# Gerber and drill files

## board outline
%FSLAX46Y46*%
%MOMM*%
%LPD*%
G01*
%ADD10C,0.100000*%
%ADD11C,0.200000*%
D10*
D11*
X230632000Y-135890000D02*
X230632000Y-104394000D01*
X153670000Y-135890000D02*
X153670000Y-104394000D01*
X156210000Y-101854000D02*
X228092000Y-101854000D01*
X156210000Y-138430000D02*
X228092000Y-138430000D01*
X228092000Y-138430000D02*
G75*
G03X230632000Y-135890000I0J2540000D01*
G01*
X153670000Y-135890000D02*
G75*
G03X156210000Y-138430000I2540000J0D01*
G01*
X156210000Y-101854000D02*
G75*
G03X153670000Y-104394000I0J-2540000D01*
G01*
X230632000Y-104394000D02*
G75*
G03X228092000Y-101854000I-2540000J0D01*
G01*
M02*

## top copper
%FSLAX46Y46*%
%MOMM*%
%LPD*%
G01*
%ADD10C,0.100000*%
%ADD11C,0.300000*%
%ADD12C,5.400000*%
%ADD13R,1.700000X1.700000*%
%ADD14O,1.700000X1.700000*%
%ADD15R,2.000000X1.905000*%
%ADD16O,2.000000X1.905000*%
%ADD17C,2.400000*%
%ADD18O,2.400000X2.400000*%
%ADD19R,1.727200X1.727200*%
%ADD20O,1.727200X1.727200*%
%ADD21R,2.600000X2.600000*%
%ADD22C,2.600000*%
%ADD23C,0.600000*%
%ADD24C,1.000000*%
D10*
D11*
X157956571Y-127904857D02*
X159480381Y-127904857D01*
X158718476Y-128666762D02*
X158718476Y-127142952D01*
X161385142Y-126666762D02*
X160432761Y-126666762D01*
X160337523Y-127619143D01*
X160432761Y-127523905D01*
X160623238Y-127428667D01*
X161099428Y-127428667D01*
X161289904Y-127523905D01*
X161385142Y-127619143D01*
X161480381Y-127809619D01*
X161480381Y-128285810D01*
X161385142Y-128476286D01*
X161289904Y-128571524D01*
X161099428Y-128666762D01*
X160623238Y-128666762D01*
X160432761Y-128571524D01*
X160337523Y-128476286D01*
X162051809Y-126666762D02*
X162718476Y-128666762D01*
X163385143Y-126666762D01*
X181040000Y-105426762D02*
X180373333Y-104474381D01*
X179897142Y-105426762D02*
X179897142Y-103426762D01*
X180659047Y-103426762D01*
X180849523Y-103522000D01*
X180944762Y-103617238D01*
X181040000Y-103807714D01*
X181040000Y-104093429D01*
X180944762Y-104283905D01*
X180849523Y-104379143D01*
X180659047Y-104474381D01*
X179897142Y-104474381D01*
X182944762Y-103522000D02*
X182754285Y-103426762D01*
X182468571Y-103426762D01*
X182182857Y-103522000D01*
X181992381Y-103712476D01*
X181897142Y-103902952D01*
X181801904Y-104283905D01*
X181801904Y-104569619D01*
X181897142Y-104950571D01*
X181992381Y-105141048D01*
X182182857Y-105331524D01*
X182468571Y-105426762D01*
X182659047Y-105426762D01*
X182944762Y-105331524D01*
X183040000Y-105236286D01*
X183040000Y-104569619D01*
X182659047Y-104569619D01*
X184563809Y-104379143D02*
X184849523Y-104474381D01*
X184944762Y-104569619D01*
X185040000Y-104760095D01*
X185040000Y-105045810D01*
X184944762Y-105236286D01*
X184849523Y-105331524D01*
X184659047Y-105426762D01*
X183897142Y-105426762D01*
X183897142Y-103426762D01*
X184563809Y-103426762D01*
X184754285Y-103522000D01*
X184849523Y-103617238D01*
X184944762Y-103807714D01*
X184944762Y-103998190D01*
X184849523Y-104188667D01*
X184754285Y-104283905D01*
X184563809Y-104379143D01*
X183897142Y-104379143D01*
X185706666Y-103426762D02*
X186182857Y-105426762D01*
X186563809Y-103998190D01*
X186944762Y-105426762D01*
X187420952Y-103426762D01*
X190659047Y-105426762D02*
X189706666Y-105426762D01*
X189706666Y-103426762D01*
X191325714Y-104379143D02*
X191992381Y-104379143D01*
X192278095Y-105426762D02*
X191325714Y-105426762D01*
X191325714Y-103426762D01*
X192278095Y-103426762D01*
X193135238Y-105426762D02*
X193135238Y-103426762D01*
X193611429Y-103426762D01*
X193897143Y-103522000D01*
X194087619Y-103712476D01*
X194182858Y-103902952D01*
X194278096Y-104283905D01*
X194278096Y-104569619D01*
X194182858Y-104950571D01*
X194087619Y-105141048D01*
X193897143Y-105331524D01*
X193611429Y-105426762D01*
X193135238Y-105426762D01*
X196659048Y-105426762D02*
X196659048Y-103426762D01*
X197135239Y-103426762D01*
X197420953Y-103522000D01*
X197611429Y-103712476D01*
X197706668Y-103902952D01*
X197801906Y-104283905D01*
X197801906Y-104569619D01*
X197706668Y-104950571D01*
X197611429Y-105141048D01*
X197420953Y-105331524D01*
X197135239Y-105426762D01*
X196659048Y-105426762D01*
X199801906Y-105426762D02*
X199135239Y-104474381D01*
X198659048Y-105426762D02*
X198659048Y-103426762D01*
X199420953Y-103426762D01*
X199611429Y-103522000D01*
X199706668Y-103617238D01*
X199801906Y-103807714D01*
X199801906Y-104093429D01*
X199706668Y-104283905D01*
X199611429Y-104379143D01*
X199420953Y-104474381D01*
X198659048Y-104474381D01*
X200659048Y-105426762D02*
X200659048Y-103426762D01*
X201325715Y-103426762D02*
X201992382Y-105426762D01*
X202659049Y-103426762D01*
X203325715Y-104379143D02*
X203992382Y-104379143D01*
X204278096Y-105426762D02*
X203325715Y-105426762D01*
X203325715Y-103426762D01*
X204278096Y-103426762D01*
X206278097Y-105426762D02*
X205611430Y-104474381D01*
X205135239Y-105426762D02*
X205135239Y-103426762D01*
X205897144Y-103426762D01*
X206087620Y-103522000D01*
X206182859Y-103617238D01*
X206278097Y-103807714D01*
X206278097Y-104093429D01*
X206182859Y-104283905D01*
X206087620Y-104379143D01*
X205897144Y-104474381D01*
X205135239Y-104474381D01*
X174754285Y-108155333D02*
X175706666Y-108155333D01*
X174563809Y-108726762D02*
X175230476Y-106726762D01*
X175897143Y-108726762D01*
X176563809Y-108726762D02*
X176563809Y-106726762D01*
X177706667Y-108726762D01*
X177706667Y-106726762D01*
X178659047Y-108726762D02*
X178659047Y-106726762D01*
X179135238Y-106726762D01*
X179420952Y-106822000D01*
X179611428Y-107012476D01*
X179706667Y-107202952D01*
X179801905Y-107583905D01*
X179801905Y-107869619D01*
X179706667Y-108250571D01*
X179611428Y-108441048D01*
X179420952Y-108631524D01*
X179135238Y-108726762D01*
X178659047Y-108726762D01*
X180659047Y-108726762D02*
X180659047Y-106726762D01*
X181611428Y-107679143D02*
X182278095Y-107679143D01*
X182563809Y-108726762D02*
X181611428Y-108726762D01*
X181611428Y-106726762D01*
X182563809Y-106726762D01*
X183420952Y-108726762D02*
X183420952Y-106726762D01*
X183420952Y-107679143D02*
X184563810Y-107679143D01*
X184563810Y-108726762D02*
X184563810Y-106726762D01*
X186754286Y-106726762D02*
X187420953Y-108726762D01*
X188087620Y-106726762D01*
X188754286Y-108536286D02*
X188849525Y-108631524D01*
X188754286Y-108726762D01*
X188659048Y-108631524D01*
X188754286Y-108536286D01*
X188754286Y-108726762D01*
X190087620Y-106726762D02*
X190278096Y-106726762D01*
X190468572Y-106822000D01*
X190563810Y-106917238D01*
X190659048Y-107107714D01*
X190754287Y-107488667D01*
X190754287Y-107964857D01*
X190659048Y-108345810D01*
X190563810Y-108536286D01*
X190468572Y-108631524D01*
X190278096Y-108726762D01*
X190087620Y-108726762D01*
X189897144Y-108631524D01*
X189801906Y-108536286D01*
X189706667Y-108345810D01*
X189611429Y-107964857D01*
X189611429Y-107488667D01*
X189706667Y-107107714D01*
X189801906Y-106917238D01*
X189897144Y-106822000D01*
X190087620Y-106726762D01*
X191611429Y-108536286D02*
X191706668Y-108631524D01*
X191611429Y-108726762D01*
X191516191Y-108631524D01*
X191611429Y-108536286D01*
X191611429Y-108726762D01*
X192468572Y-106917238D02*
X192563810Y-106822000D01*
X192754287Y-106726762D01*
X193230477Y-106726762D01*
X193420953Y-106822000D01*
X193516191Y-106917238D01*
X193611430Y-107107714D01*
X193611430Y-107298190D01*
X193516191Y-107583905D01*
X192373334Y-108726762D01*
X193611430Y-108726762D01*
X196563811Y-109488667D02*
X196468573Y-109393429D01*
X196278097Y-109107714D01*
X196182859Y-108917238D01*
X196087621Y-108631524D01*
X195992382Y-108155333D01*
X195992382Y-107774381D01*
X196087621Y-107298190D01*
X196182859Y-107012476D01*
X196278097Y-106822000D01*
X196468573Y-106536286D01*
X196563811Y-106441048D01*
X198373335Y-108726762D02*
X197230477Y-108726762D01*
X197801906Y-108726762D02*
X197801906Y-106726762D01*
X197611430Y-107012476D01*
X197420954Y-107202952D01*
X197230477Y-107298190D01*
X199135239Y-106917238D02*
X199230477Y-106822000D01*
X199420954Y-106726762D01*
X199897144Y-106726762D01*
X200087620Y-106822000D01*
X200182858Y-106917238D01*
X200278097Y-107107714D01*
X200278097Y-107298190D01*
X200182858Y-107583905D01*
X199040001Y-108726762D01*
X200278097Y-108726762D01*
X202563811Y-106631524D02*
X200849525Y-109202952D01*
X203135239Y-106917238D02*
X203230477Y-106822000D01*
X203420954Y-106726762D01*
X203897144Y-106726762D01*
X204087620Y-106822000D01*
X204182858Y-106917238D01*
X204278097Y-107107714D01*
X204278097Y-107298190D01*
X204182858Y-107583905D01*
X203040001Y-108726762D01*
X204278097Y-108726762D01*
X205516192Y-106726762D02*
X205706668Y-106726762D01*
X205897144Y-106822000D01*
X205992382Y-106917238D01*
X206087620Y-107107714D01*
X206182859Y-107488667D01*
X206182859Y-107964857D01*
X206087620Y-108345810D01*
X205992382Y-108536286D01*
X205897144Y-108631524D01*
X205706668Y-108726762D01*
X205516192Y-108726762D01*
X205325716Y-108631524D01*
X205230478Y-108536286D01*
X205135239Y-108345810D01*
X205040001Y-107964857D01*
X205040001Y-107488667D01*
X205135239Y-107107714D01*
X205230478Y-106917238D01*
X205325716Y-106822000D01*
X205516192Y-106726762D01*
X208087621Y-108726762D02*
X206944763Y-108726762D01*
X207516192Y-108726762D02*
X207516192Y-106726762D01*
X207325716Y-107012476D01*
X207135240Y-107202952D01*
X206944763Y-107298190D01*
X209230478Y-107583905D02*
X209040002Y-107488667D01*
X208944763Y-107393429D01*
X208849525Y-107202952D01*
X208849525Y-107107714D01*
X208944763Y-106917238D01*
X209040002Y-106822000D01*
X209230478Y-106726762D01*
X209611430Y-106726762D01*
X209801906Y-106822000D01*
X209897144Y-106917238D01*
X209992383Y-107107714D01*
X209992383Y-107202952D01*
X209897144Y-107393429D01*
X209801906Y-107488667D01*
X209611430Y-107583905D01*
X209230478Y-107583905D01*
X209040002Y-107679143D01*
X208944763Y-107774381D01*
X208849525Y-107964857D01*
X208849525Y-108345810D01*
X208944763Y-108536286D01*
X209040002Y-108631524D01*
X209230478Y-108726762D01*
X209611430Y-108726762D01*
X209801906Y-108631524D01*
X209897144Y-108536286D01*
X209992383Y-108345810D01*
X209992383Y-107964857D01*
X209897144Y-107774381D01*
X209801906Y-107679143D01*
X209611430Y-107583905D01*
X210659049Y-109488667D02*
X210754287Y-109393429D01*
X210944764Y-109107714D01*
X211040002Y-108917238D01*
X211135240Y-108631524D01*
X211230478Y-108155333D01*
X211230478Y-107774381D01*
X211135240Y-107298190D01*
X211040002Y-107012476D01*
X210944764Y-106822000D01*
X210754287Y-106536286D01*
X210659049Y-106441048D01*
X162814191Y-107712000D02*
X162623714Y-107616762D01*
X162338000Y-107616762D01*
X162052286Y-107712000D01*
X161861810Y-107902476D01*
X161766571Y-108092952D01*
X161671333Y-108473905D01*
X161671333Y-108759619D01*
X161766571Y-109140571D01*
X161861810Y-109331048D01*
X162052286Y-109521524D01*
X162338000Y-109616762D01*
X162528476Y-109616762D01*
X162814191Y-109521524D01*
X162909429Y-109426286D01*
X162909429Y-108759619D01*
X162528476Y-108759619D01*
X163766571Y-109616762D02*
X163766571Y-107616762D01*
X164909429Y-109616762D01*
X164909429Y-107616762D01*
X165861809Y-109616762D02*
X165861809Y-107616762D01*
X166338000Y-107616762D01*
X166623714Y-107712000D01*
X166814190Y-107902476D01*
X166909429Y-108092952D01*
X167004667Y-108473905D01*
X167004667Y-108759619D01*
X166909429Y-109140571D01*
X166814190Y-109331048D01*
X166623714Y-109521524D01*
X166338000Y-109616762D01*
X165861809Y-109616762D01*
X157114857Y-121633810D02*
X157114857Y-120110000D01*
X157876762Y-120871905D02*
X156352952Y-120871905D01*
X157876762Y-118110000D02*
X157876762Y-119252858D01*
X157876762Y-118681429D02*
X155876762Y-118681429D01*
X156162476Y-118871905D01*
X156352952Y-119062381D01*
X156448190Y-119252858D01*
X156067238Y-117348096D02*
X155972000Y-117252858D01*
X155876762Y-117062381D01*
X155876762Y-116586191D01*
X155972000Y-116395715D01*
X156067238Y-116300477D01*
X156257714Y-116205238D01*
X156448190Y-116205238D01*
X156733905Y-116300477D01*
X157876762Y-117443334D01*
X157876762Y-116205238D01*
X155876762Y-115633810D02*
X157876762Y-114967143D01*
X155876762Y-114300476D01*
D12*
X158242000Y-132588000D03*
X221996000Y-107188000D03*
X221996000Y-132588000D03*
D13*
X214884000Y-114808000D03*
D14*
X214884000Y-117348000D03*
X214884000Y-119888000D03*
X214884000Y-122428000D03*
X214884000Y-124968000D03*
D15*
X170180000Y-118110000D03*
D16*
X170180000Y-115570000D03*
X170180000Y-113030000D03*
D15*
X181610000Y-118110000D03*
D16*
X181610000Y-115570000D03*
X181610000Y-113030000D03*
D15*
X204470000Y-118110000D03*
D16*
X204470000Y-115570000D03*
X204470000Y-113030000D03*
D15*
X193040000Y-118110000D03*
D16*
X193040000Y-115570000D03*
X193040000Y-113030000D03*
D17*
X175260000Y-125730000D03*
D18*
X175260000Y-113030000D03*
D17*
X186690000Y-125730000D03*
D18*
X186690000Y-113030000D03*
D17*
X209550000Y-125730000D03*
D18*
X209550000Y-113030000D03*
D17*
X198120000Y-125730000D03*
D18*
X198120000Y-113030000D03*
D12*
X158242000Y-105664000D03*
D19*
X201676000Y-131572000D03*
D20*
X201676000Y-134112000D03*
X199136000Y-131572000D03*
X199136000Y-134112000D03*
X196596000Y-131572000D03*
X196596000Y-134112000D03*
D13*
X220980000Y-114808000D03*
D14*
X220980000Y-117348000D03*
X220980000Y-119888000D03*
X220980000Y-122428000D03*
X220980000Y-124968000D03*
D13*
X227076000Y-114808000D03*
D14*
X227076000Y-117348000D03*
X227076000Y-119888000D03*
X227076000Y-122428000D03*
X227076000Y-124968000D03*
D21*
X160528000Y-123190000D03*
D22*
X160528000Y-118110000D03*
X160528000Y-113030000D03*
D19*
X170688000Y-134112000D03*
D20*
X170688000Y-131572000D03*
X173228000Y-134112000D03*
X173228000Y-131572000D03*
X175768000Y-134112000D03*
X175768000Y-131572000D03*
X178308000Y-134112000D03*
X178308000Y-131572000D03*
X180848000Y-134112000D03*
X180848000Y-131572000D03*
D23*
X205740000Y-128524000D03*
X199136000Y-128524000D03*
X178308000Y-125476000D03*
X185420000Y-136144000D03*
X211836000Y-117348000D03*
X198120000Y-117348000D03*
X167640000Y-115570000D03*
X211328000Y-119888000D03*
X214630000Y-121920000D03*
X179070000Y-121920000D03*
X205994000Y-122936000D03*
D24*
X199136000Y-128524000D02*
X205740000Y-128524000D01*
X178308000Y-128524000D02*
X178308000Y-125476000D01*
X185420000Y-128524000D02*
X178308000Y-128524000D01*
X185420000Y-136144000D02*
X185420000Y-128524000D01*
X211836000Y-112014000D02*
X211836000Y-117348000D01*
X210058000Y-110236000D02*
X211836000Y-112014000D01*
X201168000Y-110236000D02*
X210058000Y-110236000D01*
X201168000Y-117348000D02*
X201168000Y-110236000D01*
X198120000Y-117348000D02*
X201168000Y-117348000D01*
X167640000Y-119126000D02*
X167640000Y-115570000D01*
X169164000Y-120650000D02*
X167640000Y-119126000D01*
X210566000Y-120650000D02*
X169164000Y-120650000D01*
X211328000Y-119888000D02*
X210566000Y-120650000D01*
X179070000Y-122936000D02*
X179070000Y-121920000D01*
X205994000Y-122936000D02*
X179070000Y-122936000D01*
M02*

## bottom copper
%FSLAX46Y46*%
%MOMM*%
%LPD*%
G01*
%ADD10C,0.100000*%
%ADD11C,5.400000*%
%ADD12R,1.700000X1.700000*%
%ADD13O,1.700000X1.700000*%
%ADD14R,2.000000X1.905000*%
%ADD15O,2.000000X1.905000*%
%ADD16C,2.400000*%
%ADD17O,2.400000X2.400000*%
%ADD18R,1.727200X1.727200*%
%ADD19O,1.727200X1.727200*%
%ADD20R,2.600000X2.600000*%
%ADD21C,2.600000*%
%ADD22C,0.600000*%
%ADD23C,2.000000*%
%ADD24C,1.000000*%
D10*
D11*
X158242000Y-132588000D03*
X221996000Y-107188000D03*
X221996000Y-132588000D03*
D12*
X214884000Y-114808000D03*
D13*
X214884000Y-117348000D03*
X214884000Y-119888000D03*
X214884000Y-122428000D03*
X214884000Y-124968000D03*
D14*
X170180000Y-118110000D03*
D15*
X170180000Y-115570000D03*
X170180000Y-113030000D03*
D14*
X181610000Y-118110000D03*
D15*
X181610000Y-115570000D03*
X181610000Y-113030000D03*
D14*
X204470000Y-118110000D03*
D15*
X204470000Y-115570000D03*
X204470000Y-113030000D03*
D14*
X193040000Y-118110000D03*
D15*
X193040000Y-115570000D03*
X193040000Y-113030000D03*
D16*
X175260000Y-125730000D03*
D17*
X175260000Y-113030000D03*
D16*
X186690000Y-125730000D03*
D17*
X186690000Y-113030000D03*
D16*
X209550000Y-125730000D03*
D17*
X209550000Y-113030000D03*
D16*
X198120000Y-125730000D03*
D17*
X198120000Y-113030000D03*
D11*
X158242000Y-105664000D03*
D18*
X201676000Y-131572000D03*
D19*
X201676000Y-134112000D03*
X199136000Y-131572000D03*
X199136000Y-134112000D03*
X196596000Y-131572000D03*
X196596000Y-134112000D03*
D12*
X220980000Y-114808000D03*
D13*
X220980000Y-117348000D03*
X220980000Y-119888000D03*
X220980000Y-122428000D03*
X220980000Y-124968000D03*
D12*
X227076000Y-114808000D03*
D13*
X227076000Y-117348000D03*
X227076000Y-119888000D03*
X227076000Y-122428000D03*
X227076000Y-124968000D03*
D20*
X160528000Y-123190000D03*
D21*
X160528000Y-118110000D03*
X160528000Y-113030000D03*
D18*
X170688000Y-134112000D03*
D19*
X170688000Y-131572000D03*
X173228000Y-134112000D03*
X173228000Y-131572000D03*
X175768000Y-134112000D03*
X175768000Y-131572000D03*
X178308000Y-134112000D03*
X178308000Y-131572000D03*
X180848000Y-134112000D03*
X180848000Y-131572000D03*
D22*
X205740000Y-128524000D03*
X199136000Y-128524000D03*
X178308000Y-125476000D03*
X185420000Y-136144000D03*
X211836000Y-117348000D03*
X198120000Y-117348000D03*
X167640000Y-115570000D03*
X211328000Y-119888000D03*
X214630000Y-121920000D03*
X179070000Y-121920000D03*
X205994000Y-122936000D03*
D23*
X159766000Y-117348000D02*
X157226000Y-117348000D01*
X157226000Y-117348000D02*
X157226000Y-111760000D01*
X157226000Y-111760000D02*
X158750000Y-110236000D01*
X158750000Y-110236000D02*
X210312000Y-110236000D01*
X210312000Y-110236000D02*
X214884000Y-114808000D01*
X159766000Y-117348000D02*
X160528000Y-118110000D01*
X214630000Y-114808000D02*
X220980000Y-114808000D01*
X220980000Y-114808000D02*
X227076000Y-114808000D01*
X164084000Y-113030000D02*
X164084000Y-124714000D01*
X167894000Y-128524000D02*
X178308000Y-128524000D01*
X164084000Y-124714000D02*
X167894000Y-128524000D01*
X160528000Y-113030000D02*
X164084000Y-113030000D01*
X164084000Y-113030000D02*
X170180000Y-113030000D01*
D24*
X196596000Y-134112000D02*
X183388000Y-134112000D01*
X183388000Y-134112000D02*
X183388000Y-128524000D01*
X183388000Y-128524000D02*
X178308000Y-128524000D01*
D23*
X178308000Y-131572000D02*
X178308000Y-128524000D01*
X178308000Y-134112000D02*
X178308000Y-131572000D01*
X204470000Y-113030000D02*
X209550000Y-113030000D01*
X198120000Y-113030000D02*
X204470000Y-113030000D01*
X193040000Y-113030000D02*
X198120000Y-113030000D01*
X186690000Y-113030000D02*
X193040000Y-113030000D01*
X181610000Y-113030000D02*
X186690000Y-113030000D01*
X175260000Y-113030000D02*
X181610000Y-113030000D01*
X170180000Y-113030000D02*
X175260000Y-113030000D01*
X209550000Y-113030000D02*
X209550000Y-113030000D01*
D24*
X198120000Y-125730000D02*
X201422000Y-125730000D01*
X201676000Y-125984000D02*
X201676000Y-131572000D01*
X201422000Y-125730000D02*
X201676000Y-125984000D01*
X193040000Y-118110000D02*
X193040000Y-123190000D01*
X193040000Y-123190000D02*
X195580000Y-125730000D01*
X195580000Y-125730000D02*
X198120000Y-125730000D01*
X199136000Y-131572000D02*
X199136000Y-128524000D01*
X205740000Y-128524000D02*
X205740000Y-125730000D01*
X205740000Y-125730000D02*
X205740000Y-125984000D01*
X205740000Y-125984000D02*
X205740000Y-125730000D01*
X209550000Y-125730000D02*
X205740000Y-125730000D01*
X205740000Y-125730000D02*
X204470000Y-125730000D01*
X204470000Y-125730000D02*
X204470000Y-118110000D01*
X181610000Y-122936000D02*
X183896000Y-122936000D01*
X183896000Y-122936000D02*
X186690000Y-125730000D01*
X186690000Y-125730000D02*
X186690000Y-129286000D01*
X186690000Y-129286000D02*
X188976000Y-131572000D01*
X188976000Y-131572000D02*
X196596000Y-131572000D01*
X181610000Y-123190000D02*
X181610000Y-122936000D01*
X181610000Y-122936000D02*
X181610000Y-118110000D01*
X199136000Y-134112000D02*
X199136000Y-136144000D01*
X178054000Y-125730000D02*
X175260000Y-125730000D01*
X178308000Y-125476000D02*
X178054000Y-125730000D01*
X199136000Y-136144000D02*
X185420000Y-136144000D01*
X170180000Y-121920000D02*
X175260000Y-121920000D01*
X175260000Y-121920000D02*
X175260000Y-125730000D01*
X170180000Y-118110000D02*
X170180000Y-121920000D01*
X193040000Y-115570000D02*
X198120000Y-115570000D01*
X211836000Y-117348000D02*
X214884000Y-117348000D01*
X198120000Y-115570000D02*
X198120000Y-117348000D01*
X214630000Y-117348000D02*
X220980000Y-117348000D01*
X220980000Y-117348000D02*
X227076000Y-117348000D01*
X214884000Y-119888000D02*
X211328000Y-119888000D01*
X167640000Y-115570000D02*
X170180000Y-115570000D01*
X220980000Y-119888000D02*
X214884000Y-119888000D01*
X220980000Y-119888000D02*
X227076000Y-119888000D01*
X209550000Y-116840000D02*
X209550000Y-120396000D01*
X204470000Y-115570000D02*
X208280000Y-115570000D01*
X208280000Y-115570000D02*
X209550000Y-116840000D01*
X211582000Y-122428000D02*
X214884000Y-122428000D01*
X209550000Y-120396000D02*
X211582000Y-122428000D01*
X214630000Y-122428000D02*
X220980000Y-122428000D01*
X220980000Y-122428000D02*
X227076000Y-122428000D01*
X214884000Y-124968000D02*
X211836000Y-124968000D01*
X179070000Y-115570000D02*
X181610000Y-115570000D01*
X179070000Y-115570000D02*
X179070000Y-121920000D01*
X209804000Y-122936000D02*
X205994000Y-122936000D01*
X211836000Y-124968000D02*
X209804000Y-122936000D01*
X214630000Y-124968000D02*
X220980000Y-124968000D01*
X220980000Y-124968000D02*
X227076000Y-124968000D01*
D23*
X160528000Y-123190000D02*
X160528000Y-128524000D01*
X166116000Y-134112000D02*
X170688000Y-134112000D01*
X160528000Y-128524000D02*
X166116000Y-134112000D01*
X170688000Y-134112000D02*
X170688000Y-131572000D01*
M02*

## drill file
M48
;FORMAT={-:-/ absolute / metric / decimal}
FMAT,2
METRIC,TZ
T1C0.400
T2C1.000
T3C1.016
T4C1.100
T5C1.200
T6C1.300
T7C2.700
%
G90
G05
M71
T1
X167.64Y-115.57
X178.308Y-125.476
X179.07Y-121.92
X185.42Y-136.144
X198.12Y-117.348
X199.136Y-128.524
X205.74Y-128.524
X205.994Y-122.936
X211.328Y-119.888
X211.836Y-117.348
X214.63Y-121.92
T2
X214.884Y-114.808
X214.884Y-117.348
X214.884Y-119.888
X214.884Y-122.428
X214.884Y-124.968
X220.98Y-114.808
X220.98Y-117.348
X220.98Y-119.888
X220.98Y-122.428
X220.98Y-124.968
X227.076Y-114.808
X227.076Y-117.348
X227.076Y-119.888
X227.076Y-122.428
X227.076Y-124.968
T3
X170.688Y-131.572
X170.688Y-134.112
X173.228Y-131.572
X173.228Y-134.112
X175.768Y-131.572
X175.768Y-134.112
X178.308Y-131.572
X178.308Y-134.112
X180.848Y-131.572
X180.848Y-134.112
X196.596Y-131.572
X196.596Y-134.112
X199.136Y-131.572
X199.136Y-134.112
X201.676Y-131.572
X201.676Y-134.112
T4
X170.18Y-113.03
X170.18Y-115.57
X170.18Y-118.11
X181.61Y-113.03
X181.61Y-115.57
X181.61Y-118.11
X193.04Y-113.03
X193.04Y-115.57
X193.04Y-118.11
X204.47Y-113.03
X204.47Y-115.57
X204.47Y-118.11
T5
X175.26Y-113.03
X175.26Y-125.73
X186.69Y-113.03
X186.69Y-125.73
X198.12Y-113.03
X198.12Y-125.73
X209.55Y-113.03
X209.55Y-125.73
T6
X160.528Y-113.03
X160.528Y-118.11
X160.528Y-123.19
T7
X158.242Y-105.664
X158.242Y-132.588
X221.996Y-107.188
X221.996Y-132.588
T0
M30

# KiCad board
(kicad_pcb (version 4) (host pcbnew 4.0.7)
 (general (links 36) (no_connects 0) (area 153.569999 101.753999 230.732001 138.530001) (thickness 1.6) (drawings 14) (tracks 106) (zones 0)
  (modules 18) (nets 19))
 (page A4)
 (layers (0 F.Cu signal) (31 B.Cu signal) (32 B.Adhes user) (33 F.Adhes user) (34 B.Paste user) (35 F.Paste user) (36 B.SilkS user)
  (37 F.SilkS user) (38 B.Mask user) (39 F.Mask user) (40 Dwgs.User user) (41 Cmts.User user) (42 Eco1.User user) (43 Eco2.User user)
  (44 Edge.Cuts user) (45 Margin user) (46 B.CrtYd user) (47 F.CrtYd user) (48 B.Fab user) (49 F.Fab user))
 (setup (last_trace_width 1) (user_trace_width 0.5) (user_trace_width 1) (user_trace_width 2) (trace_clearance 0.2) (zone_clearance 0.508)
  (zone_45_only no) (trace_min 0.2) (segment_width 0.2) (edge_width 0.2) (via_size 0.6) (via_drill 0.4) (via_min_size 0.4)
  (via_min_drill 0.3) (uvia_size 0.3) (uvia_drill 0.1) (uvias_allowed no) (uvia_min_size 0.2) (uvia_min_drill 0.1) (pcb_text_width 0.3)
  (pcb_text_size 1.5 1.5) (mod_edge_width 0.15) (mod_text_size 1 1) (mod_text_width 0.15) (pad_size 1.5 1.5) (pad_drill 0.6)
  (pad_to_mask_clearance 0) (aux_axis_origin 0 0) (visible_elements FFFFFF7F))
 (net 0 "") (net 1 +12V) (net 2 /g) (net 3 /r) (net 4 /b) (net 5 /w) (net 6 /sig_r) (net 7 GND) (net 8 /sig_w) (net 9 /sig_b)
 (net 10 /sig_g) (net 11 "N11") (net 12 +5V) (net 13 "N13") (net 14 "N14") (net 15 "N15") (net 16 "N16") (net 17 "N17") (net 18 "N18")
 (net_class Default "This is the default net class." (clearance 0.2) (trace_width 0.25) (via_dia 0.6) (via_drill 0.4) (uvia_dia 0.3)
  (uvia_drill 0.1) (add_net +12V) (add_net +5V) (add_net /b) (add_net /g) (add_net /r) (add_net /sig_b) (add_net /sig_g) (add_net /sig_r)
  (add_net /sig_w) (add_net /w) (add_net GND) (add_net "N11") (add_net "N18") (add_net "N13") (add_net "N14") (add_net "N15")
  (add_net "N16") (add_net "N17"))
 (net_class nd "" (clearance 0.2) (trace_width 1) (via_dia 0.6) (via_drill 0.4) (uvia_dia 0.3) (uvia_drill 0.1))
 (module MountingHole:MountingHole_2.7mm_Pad (layer F.Cu) (at 158.242 132.588)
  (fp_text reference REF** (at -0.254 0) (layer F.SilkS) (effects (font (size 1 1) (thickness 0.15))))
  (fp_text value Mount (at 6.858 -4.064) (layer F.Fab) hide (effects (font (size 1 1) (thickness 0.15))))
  (pad 1 thru_hole circle (at 0 0) (size 5.4 5.4) (drill 2.7) (layers *.Cu *.Mask)))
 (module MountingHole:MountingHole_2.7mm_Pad (layer F.Cu) (at 221.996 107.188)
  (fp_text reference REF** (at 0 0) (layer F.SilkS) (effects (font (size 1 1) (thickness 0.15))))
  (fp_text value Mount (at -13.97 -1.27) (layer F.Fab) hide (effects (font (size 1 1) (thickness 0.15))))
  (pad 1 thru_hole circle (at 0 0) (size 5.4 5.4) (drill 2.7) (layers *.Cu *.Mask)))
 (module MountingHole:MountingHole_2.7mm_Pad (layer F.Cu) (at 221.996 132.588)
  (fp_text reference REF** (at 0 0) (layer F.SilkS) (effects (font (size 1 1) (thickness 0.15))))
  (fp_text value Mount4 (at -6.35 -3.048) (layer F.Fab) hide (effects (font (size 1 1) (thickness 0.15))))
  (pad 1 thru_hole circle (at 0 0) (size 5.4 5.4) (drill 2.7) (layers *.Cu *.Mask)))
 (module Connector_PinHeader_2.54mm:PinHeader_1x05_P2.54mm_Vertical (layer F.Cu) (at 214.884 114.808)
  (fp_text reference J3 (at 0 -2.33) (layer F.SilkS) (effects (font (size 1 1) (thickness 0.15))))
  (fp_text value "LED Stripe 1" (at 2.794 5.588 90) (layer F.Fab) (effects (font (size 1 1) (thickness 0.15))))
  (pad 1 thru_hole rect (at 0 0) (size 1.7 1.7) (drill 1) (layers *.Cu *.Mask) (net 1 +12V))
  (pad 2 thru_hole oval (at 0 2.54) (size 1.7 1.7) (drill 1) (layers *.Cu *.Mask) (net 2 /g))
  (pad 3 thru_hole oval (at 0 5.08) (size 1.7 1.7) (drill 1) (layers *.Cu *.Mask) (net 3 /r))
  (pad 4 thru_hole oval (at 0 7.62) (size 1.7 1.7) (drill 1) (layers *.Cu *.Mask) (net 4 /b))
  (pad 5 thru_hole oval (at 0 10.16) (size 1.7 1.7) (drill 1) (layers *.Cu *.Mask) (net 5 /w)))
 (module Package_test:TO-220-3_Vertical (layer F.Cu) (at 170.18 118.11 90)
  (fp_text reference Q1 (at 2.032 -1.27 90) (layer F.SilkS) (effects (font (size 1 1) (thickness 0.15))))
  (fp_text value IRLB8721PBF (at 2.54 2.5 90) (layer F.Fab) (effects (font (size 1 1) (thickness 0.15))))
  (pad 1 thru_hole rect (at 0 0 90) (size 1.905 2) (drill 1.1) (layers *.Cu *.Mask) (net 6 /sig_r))
  (pad 2 thru_hole oval (at 2.54 0 90) (size 1.905 2) (drill 1.1) (layers *.Cu *.Mask) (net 3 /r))
  (pad 3 thru_hole oval (at 5.08 0 90) (size 1.905 2) (drill 1.1) (layers *.Cu *.Mask) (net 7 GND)))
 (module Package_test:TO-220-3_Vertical (layer F.Cu) (at 181.61 118.11 90)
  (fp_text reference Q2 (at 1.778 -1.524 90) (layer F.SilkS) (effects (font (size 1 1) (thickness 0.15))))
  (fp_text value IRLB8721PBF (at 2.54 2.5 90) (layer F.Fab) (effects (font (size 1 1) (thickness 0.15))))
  (pad 1 thru_hole rect (at 0 0 90) (size 1.905 2) (drill 1.1) (layers *.Cu *.Mask) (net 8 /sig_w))
  (pad 2 thru_hole oval (at 2.54 0 90) (size 1.905 2) (drill 1.1) (layers *.Cu *.Mask) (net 5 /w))
  (pad 3 thru_hole oval (at 5.08 0 90) (size 1.905 2) (drill 1.1) (layers *.Cu *.Mask) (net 7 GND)))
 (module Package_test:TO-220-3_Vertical (layer F.Cu) (at 204.47 118.11 90)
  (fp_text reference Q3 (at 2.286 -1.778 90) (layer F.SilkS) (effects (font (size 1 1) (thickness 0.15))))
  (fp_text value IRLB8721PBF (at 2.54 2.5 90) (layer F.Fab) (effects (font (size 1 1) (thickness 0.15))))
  (pad 1 thru_hole rect (at 0 0 90) (size 1.905 2) (drill 1.1) (layers *.Cu *.Mask) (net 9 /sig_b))
  (pad 2 thru_hole oval (at 2.54 0 90) (size 1.905 2) (drill 1.1) (layers *.Cu *.Mask) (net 4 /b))
  (pad 3 thru_hole oval (at 5.08 0 90) (size 1.905 2) (drill 1.1) (layers *.Cu *.Mask) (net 7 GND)))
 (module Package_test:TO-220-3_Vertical (layer F.Cu) (at 193.04 118.11 90)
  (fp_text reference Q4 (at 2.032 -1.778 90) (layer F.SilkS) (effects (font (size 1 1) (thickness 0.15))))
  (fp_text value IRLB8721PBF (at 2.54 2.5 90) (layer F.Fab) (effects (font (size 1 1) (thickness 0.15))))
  (pad 1 thru_hole rect (at 0 0 90) (size 1.905 2) (drill 1.1) (layers *.Cu *.Mask) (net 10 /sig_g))
  (pad 2 thru_hole oval (at 2.54 0 90) (size 1.905 2) (drill 1.1) (layers *.Cu *.Mask) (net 2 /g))
  (pad 3 thru_hole oval (at 5.08 0 90) (size 1.905 2) (drill 1.1) (layers *.Cu *.Mask) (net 7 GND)))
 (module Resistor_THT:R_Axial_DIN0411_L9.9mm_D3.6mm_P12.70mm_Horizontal (layer F.Cu) (at 175.26 125.73 90)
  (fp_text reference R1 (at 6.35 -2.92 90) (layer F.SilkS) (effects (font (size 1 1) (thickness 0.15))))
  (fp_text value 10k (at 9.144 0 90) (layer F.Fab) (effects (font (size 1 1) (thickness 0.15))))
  (pad 1 thru_hole circle (at 0 0 90) (size 2.4 2.4) (drill 1.2) (layers *.Cu *.Mask) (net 6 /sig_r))
  (pad 2 thru_hole oval (at 12.7 0 90) (size 2.4 2.4) (drill 1.2) (layers *.Cu *.Mask) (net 7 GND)))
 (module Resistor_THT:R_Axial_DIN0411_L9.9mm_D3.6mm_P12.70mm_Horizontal (layer F.Cu) (at 186.69 125.73 90)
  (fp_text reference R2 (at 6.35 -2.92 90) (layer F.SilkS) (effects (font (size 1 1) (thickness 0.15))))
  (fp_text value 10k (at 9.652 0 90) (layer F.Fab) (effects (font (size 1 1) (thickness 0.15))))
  (pad 1 thru_hole circle (at 0 0 90) (size 2.4 2.4) (drill 1.2) (layers *.Cu *.Mask) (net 8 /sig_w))
  (pad 2 thru_hole oval (at 12.7 0 90) (size 2.4 2.4) (drill 1.2) (layers *.Cu *.Mask) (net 7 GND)))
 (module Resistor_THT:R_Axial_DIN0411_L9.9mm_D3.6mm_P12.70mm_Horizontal (layer F.Cu) (at 209.55 125.73 90)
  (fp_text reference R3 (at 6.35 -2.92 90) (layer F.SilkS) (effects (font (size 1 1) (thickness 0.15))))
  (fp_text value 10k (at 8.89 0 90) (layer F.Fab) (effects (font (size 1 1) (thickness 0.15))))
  (pad 1 thru_hole circle (at 0 0 90) (size 2.4 2.4) (drill 1.2) (layers *.Cu *.Mask) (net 9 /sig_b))
  (pad 2 thru_hole oval (at 12.7 0 90) (size 2.4 2.4) (drill 1.2) (layers *.Cu *.Mask) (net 7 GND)))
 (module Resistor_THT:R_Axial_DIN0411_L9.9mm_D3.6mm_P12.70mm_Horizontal (layer F.Cu) (at 198.12 125.73 90)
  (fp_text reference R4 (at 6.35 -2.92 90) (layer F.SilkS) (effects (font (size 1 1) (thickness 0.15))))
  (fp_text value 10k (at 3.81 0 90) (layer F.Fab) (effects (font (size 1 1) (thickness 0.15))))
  (pad 1 thru_hole circle (at 0 0 90) (size 2.4 2.4) (drill 1.2) (layers *.Cu *.Mask) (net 10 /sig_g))
  (pad 2 thru_hole oval (at 12.7 0 90) (size 2.4 2.4) (drill 1.2) (layers *.Cu *.Mask) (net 7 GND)))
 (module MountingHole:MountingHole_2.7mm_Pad (layer F.Cu) (at 158.242 105.664)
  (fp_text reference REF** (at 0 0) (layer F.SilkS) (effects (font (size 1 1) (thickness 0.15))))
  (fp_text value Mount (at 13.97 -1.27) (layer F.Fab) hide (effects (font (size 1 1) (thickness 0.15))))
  (pad 1 thru_hole circle (at 0 0) (size 5.4 5.4) (drill 2.7) (layers *.Cu *.Mask)))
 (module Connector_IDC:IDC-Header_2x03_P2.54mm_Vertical (layer F.Cu) (at 201.676 131.572 270)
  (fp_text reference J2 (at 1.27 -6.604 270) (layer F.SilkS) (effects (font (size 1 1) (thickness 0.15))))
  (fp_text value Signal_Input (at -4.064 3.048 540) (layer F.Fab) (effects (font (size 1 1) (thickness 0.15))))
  (pad 1 thru_hole rect (at 0 0 270) (size 1.7272 1.7272) (drill 1.016) (layers *.Cu *.Mask) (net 10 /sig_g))
  (pad 2 thru_hole oval (at 2.54 0 270) (size 1.7272 1.7272) (drill 1.016) (layers *.Cu *.Mask) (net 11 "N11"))
  (pad 3 thru_hole oval (at 0 2.54 270) (size 1.7272 1.7272) (drill 1.016) (layers *.Cu *.Mask) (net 9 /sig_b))
  (pad 4 thru_hole oval (at 2.54 2.54 270) (size 1.7272 1.7272) (drill 1.016) (layers *.Cu *.Mask) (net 6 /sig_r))
  (pad 5 thru_hole oval (at 0 5.08 270) (size 1.7272 1.7272) (drill 1.016) (layers *.Cu *.Mask) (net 8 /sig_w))
  (pad 6 thru_hole oval (at 2.54 5.08 270) (size 1.7272 1.7272) (drill 1.016) (layers *.Cu *.Mask) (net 7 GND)))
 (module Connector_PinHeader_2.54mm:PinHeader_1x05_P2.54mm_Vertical (layer F.Cu) (at 220.98 114.808)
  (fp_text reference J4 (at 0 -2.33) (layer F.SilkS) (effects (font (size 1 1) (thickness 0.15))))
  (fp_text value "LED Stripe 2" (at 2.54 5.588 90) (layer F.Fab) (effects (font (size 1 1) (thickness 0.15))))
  (pad 1 thru_hole rect (at 0 0) (size 1.7 1.7) (drill 1) (layers *.Cu *.Mask) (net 1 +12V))
  (pad 2 thru_hole oval (at 0 2.54) (size 1.7 1.7) (drill 1) (layers *.Cu *.Mask) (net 2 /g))
  (pad 3 thru_hole oval (at 0 5.08) (size 1.7 1.7) (drill 1) (layers *.Cu *.Mask) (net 3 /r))
  (pad 4 thru_hole oval (at 0 7.62) (size 1.7 1.7) (drill 1) (layers *.Cu *.Mask) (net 4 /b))
  (pad 5 thru_hole oval (at 0 10.16) (size 1.7 1.7) (drill 1) (layers *.Cu *.Mask) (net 5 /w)))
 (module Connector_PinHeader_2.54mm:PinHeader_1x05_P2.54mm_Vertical (layer F.Cu) (at 227.076 114.808)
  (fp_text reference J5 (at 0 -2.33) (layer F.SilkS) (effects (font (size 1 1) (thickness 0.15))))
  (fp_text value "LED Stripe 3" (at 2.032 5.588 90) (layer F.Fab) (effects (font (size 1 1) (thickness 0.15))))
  (pad 1 thru_hole rect (at 0 0) (size 1.7 1.7) (drill 1) (layers *.Cu *.Mask) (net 1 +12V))
  (pad 2 thru_hole oval (at 0 2.54) (size 1.7 1.7) (drill 1) (layers *.Cu *.Mask) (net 2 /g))
  (pad 3 thru_hole oval (at 0 5.08) (size 1.7 1.7) (drill 1) (layers *.Cu *.Mask) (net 3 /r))
  (pad 4 thru_hole oval (at 0 7.62) (size 1.7 1.7) (drill 1) (layers *.Cu *.Mask) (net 4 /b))
  (pad 5 thru_hole oval (at 0 10.16) (size 1.7 1.7) (drill 1) (layers *.Cu *.Mask) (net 5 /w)))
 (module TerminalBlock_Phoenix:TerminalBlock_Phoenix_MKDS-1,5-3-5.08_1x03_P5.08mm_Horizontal (layer F.Cu) (at 160.528 123.19 90)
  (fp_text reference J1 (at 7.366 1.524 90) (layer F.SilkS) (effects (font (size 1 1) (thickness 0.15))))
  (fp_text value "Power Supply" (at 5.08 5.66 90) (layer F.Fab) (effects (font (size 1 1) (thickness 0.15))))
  (pad 1 thru_hole rect (at 0 0 90) (size 2.6 2.6) (drill 1.3) (layers *.Cu *.Mask) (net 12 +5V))
  (pad 2 thru_hole circle (at 5.08 0 90) (size 2.6 2.6) (drill 1.3) (layers *.Cu *.Mask) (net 1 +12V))
  (pad 3 thru_hole circle (at 10.16 0 90) (size 2.6 2.6) (drill 1.3) (layers *.Cu *.Mask) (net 7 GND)))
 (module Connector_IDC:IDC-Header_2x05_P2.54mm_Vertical (layer F.Cu) (at 170.688 134.112 90)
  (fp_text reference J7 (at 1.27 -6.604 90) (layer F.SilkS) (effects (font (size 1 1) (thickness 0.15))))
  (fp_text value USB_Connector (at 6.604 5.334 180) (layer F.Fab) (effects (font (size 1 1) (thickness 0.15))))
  (pad 1 thru_hole rect (at 0 0 90) (size 1.7272 1.7272) (drill 1.016) (layers *.Cu *.Mask) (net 12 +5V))
  (pad 2 thru_hole oval (at 2.54 0 90) (size 1.7272 1.7272) (drill 1.016) (layers *.Cu *.Mask) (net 12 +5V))
  (pad 3 thru_hole oval (at 0 2.54 90) (size 1.7272 1.7272) (drill 1.016) (layers *.Cu *.Mask) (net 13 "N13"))
  (pad 4 thru_hole oval (at 2.54 2.54 90) (size 1.7272 1.7272) (drill 1.016) (layers *.Cu *.Mask) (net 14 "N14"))
  (pad 5 thru_hole oval (at 0 5.08 90) (size 1.7272 1.7272) (drill 1.016) (layers *.Cu *.Mask) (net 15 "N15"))
  (pad 6 thru_hole oval (at 2.54 5.08 90) (size 1.7272 1.7272) (drill 1.016) (layers *.Cu *.Mask) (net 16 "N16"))
  (pad 7 thru_hole oval (at 0 7.62 90) (size 1.7272 1.7272) (drill 1.016) (layers *.Cu *.Mask) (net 7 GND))
  (pad 8 thru_hole oval (at 2.54 7.62 90) (size 1.7272 1.7272) (drill 1.016) (layers *.Cu *.Mask) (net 7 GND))
  (pad 9 thru_hole oval (at 0 10.16 90) (size 1.7272 1.7272) (drill 1.016) (layers *.Cu *.Mask) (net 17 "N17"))
  (pad 10 thru_hole oval (at 2.54 10.16 90) (size 1.7272 1.7272) (drill 1.016) (layers *.Cu *.Mask) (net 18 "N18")))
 (gr_line (start 230.632 135.89) (end 230.632 104.394) (angle 90) (layer Edge.Cuts) (width 0.2))
 (gr_line (start 153.67 135.89) (end 153.67 104.394) (angle 90) (layer Edge.Cuts) (width 0.2))
 (gr_line (start 156.21 101.854) (end 228.092 101.854) (angle 90) (layer Edge.Cuts) (width 0.2))
 (gr_line (start 156.21 138.43) (end 228.092 138.43) (angle 90) (layer Edge.Cuts) (width 0.2))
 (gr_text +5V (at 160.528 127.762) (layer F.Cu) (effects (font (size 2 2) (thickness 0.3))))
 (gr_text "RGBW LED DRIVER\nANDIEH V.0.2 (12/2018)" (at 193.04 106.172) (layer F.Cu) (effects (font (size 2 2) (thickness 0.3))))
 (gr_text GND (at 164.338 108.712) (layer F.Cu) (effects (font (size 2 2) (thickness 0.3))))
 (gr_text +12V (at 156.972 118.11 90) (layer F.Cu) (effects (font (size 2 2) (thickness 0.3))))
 (gr_arc (start 228.092 135.89) (end 230.632 135.89) (angle 90) (layer Edge.Cuts) (width 0.2))
 (gr_arc (start 156.21 135.89) (end 156.21 138.43) (angle 90) (layer Edge.Cuts) (width 0.2))
 (gr_arc (start 156.21 104.394) (end 153.67 104.394) (angle 90) (layer Edge.Cuts) (width 0.2))
 (gr_arc (start 228.092 104.394) (end 228.092 101.854) (angle 90) (layer Edge.Cuts) (width 0.2))
 (segment (start 159.766 117.348) (end 157.226 117.348) (width 2) (layer B.Cu) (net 1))
 (segment (start 157.226 117.348) (end 157.226 111.76) (width 2) (layer B.Cu) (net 1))
 (segment (start 157.226 111.76) (end 158.75 110.236) (width 2) (layer B.Cu) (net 1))
 (segment (start 158.75 110.236) (end 210.312 110.236) (width 2) (layer B.Cu) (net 1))
 (segment (start 210.312 110.236) (end 214.884 114.808) (width 2) (layer B.Cu) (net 1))
 (segment (start 159.766 117.348) (end 160.528 118.11) (width 2) (layer B.Cu) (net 1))
 (segment (start 214.63 114.808) (end 220.98 114.808) (width 2) (layer B.Cu) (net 1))
 (segment (start 220.98 114.808) (end 227.076 114.808) (width 2) (layer B.Cu) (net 1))
 (segment (start 164.084 113.03) (end 164.084 124.714) (width 2) (layer B.Cu) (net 7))
 (segment (start 167.894 128.524) (end 178.308 128.524) (width 2) (layer B.Cu) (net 7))
 (segment (start 164.084 124.714) (end 167.894 128.524) (width 2) (layer B.Cu) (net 7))
 (segment (start 160.528 113.03) (end 164.084 113.03) (width 2) (layer B.Cu) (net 7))
 (segment (start 164.084 113.03) (end 170.18 113.03) (width 2) (layer B.Cu) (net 7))
 (segment (start 196.596 134.112) (end 183.388 134.112) (width 1) (layer B.Cu) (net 7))
 (segment (start 183.388 134.112) (end 183.388 128.524) (width 1) (layer B.Cu) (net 7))
 (segment (start 183.388 128.524) (end 178.308 128.524) (width 1) (layer B.Cu) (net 7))
 (segment (start 178.308 131.572) (end 178.308 128.524) (width 2) (layer B.Cu) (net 7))
 (segment (start 178.308 134.112) (end 178.308 131.572) (width 2) (layer B.Cu) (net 7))
 (segment (start 204.47 113.03) (end 209.55 113.03) (width 2) (layer B.Cu) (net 7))
 (segment (start 198.12 113.03) (end 204.47 113.03) (width 2) (layer B.Cu) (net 7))
 (segment (start 193.04 113.03) (end 198.12 113.03) (width 2) (layer B.Cu) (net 7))
 (segment (start 186.69 113.03) (end 193.04 113.03) (width 2) (layer B.Cu) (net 7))
 (segment (start 181.61 113.03) (end 186.69 113.03) (width 2) (layer B.Cu) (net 7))
 (segment (start 175.26 113.03) (end 181.61 113.03) (width 2) (layer B.Cu) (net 7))
 (segment (start 170.18 113.03) (end 175.26 113.03) (width 2) (layer B.Cu) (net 7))
 (segment (start 209.55 113.03) (end 209.55 113.03) (width 2) (layer B.Cu) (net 7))
 (segment (start 198.12 125.73) (end 201.422 125.73) (width 1) (layer B.Cu) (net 10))
 (segment (start 201.676 125.984) (end 201.676 131.572) (width 1) (layer B.Cu) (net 10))
 (segment (start 201.422 125.73) (end 201.676 125.984) (width 1) (layer B.Cu) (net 10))
 (segment (start 193.04 118.11) (end 193.04 123.19) (width 1) (layer B.Cu) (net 10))
 (segment (start 193.04 123.19) (end 195.58 125.73) (width 1) (layer B.Cu) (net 10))
 (segment (start 195.58 125.73) (end 198.12 125.73) (width 1) (layer B.Cu) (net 10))
 (segment (start 199.136 131.572) (end 199.136 128.524) (width 1) (layer B.Cu) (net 9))
 (segment (start 205.74 128.524) (end 205.74 125.73) (width 1) (layer B.Cu) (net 9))
 (via (at 205.74 128.524) (size 0.6) (drill 0.4) (layers F.Cu B.Cu) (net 9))
 (segment (start 199.136 128.524) (end 205.74 128.524) (width 1) (layer F.Cu) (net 9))
 (via (at 199.136 128.524) (size 0.6) (drill 0.4) (layers F.Cu B.Cu) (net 9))
 (segment (start 205.74 125.73) (end 205.74 125.984) (width 1) (layer B.Cu) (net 9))
 (segment (start 205.74 125.984) (end 205.74 125.73) (width 1) (layer B.Cu) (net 9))
 (segment (start 209.55 125.73) (end 205.74 125.73) (width 1) (layer B.Cu) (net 9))
 (segment (start 205.74 125.73) (end 204.47 125.73) (width 1) (layer B.Cu) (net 9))
 (segment (start 204.47 125.73) (end 204.47 118.11) (width 1) (layer B.Cu) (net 9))
 (segment (start 181.61 122.936) (end 183.896 122.936) (width 1) (layer B.Cu) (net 8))
 (segment (start 183.896 122.936) (end 186.69 125.73) (width 1) (layer B.Cu) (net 8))
 (segment (start 186.69 125.73) (end 186.69 129.286) (width 1) (layer B.Cu) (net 8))
 (segment (start 186.69 129.286) (end 188.976 131.572) (width 1) (layer B.Cu) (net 8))
 (segment (start 188.976 131.572) (end 196.596 131.572) (width 1) (layer B.Cu) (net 8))
 (segment (start 181.61 123.19) (end 181.61 122.936) (width 1) (layer B.Cu) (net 8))
 (segment (start 181.61 122.936) (end 181.61 118.11) (width 1) (layer B.Cu) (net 8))
 (segment (start 199.136 134.112) (end 199.136 136.144) (width 1) (layer B.Cu) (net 6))
 (segment (start 178.054 125.73) (end 175.26 125.73) (width 1) (layer B.Cu) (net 6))
 (segment (start 178.308 125.476) (end 178.054 125.73) (width 1) (layer B.Cu) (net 6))
 (via (at 178.308 125.476) (size 0.6) (drill 0.4) (layers F.Cu B.Cu) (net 6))
 (segment (start 178.308 128.524) (end 178.308 125.476) (width 1) (layer F.Cu) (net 6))
 (segment (start 185.42 128.524) (end 178.308 128.524) (width 1) (layer F.Cu) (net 6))
 (segment (start 185.42 136.144) (end 185.42 128.524) (width 1) (layer F.Cu) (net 6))
 (via (at 185.42 136.144) (size 0.6) (drill 0.4) (layers F.Cu B.Cu) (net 6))
 (segment (start 199.136 136.144) (end 185.42 136.144) (width 1) (layer B.Cu) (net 6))
 (segment (start 170.18 121.92) (end 175.26 121.92) (width 1) (layer B.Cu) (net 6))
 (segment (start 175.26 121.92) (end 175.26 125.73) (width 1) (layer B.Cu) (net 6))
 (segment (start 170.18 118.11) (end 170.18 121.92) (width 1) (layer B.Cu) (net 6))
 (segment (start 193.04 115.57) (end 198.12 115.57) (width 1) (layer B.Cu) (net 2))
 (segment (start 211.836 117.348) (end 214.884 117.348) (width 1) (layer B.Cu) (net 2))
 (via (at 211.836 117.348) (size 0.6) (drill 0.4) (layers F.Cu B.Cu) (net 2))
 (segment (start 211.836 112.014) (end 211.836 117.348) (width 1) (layer F.Cu) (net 2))
 (segment (start 210.058 110.236) (end 211.836 112.014) (width 1) (layer F.Cu) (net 2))
 (segment (start 201.168 110.236) (end 210.058 110.236) (width 1) (layer F.Cu) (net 2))
 (segment (start 201.168 117.348) (end 201.168 110.236) (width 1) (layer F.Cu) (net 2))
 (segment (start 198.12 117.348) (end 201.168 117.348) (width 1) (layer F.Cu) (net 2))
 (via (at 198.12 117.348) (size 0.6) (drill 0.4) (layers F.Cu B.Cu) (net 2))
 (segment (start 198.12 115.57) (end 198.12 117.348) (width 1) (layer B.Cu) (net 2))
 (segment (start 214.63 117.348) (end 220.98 117.348) (width 1) (layer B.Cu) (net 2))
 (segment (start 220.98 117.348) (end 227.076 117.348) (width 1) (layer B.Cu) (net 2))
 (segment (start 214.884 119.888) (end 211.328 119.888) (width 1) (layer B.Cu) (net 3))
 (segment (start 167.64 115.57) (end 170.18 115.57) (width 1) (layer B.Cu) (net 3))
 (via (at 167.64 115.57) (size 0.6) (drill 0.4) (layers F.Cu B.Cu) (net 3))
 (segment (start 167.64 119.126) (end 167.64 115.57) (width 1) (layer F.Cu) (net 3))
 (segment (start 169.164 120.65) (end 167.64 119.126) (width 1) (layer F.Cu) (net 3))
 (segment (start 210.566 120.65) (end 169.164 120.65) (width 1) (layer F.Cu) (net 3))
 (segment (start 211.328 119.888) (end 210.566 120.65) (width 1) (layer F.Cu) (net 3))
 (via (at 211.328 119.888) (size 0.6) (drill 0.4) (layers F.Cu B.Cu) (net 3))
 (segment (start 220.98 119.888) (end 214.884 119.888) (width 1) (layer B.Cu) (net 3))
 (segment (start 220.98 119.888) (end 227.076 119.888) (width 1) (layer B.Cu) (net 3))
 (segment (start 209.55 116.84) (end 209.55 120.396) (width 1) (layer B.Cu) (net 4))
 (segment (start 204.47 115.57) (end 208.28 115.57) (width 1) (layer B.Cu) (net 4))
 (segment (start 208.28 115.57) (end 209.55 116.84) (width 1) (layer B.Cu) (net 4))
 (segment (start 211.582 122.428) (end 214.884 122.428) (width 1) (layer B.Cu) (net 4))
 (segment (start 209.55 120.396) (end 211.582 122.428) (width 1) (layer B.Cu) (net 4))
 (segment (start 214.63 122.428) (end 220.98 122.428) (width 1) (layer B.Cu) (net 4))
 (segment (start 220.98 122.428) (end 227.076 122.428) (width 1) (layer B.Cu) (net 4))
 (via (at 214.63 121.92) (size 0.6) (drill 0.4) (layers F.Cu B.Cu) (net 4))
 (segment (start 214.884 124.968) (end 211.836 124.968) (width 1) (layer B.Cu) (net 5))
 (segment (start 179.07 115.57) (end 181.61 115.57) (width 1) (layer B.Cu) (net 5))
 (segment (start 179.07 115.57) (end 179.07 121.92) (width 1) (layer B.Cu) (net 5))
 (via (at 179.07 121.92) (size 0.6) (drill 0.4) (layers F.Cu B.Cu) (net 5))
 (segment (start 179.07 122.936) (end 179.07 121.92) (width 1) (layer F.Cu) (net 5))
 (segment (start 205.994 122.936) (end 179.07 122.936) (width 1) (layer F.Cu) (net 5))
 (via (at 205.994 122.936) (size 0.6) (drill 0.4) (layers F.Cu B.Cu) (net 5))
 (segment (start 209.804 122.936) (end 205.994 122.936) (width 1) (layer B.Cu) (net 5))
 (segment (start 211.836 124.968) (end 209.804 122.936) (width 1) (layer B.Cu) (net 5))
 (segment (start 214.63 124.968) (end 220.98 124.968) (width 1) (layer B.Cu) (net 5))
 (segment (start 220.98 124.968) (end 227.076 124.968) (width 1) (layer B.Cu) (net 5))
 (segment (start 160.528 123.19) (end 160.528 128.524) (width 2) (layer B.Cu) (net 12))
 (segment (start 166.116 134.112) (end 170.688 134.112) (width 2) (layer B.Cu) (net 12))
 (segment (start 160.528 128.524) (end 166.116 134.112) (width 2) (layer B.Cu) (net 12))
 (segment (start 170.688 134.112) (end 170.688 131.572) (width 2) (layer B.Cu) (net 12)))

